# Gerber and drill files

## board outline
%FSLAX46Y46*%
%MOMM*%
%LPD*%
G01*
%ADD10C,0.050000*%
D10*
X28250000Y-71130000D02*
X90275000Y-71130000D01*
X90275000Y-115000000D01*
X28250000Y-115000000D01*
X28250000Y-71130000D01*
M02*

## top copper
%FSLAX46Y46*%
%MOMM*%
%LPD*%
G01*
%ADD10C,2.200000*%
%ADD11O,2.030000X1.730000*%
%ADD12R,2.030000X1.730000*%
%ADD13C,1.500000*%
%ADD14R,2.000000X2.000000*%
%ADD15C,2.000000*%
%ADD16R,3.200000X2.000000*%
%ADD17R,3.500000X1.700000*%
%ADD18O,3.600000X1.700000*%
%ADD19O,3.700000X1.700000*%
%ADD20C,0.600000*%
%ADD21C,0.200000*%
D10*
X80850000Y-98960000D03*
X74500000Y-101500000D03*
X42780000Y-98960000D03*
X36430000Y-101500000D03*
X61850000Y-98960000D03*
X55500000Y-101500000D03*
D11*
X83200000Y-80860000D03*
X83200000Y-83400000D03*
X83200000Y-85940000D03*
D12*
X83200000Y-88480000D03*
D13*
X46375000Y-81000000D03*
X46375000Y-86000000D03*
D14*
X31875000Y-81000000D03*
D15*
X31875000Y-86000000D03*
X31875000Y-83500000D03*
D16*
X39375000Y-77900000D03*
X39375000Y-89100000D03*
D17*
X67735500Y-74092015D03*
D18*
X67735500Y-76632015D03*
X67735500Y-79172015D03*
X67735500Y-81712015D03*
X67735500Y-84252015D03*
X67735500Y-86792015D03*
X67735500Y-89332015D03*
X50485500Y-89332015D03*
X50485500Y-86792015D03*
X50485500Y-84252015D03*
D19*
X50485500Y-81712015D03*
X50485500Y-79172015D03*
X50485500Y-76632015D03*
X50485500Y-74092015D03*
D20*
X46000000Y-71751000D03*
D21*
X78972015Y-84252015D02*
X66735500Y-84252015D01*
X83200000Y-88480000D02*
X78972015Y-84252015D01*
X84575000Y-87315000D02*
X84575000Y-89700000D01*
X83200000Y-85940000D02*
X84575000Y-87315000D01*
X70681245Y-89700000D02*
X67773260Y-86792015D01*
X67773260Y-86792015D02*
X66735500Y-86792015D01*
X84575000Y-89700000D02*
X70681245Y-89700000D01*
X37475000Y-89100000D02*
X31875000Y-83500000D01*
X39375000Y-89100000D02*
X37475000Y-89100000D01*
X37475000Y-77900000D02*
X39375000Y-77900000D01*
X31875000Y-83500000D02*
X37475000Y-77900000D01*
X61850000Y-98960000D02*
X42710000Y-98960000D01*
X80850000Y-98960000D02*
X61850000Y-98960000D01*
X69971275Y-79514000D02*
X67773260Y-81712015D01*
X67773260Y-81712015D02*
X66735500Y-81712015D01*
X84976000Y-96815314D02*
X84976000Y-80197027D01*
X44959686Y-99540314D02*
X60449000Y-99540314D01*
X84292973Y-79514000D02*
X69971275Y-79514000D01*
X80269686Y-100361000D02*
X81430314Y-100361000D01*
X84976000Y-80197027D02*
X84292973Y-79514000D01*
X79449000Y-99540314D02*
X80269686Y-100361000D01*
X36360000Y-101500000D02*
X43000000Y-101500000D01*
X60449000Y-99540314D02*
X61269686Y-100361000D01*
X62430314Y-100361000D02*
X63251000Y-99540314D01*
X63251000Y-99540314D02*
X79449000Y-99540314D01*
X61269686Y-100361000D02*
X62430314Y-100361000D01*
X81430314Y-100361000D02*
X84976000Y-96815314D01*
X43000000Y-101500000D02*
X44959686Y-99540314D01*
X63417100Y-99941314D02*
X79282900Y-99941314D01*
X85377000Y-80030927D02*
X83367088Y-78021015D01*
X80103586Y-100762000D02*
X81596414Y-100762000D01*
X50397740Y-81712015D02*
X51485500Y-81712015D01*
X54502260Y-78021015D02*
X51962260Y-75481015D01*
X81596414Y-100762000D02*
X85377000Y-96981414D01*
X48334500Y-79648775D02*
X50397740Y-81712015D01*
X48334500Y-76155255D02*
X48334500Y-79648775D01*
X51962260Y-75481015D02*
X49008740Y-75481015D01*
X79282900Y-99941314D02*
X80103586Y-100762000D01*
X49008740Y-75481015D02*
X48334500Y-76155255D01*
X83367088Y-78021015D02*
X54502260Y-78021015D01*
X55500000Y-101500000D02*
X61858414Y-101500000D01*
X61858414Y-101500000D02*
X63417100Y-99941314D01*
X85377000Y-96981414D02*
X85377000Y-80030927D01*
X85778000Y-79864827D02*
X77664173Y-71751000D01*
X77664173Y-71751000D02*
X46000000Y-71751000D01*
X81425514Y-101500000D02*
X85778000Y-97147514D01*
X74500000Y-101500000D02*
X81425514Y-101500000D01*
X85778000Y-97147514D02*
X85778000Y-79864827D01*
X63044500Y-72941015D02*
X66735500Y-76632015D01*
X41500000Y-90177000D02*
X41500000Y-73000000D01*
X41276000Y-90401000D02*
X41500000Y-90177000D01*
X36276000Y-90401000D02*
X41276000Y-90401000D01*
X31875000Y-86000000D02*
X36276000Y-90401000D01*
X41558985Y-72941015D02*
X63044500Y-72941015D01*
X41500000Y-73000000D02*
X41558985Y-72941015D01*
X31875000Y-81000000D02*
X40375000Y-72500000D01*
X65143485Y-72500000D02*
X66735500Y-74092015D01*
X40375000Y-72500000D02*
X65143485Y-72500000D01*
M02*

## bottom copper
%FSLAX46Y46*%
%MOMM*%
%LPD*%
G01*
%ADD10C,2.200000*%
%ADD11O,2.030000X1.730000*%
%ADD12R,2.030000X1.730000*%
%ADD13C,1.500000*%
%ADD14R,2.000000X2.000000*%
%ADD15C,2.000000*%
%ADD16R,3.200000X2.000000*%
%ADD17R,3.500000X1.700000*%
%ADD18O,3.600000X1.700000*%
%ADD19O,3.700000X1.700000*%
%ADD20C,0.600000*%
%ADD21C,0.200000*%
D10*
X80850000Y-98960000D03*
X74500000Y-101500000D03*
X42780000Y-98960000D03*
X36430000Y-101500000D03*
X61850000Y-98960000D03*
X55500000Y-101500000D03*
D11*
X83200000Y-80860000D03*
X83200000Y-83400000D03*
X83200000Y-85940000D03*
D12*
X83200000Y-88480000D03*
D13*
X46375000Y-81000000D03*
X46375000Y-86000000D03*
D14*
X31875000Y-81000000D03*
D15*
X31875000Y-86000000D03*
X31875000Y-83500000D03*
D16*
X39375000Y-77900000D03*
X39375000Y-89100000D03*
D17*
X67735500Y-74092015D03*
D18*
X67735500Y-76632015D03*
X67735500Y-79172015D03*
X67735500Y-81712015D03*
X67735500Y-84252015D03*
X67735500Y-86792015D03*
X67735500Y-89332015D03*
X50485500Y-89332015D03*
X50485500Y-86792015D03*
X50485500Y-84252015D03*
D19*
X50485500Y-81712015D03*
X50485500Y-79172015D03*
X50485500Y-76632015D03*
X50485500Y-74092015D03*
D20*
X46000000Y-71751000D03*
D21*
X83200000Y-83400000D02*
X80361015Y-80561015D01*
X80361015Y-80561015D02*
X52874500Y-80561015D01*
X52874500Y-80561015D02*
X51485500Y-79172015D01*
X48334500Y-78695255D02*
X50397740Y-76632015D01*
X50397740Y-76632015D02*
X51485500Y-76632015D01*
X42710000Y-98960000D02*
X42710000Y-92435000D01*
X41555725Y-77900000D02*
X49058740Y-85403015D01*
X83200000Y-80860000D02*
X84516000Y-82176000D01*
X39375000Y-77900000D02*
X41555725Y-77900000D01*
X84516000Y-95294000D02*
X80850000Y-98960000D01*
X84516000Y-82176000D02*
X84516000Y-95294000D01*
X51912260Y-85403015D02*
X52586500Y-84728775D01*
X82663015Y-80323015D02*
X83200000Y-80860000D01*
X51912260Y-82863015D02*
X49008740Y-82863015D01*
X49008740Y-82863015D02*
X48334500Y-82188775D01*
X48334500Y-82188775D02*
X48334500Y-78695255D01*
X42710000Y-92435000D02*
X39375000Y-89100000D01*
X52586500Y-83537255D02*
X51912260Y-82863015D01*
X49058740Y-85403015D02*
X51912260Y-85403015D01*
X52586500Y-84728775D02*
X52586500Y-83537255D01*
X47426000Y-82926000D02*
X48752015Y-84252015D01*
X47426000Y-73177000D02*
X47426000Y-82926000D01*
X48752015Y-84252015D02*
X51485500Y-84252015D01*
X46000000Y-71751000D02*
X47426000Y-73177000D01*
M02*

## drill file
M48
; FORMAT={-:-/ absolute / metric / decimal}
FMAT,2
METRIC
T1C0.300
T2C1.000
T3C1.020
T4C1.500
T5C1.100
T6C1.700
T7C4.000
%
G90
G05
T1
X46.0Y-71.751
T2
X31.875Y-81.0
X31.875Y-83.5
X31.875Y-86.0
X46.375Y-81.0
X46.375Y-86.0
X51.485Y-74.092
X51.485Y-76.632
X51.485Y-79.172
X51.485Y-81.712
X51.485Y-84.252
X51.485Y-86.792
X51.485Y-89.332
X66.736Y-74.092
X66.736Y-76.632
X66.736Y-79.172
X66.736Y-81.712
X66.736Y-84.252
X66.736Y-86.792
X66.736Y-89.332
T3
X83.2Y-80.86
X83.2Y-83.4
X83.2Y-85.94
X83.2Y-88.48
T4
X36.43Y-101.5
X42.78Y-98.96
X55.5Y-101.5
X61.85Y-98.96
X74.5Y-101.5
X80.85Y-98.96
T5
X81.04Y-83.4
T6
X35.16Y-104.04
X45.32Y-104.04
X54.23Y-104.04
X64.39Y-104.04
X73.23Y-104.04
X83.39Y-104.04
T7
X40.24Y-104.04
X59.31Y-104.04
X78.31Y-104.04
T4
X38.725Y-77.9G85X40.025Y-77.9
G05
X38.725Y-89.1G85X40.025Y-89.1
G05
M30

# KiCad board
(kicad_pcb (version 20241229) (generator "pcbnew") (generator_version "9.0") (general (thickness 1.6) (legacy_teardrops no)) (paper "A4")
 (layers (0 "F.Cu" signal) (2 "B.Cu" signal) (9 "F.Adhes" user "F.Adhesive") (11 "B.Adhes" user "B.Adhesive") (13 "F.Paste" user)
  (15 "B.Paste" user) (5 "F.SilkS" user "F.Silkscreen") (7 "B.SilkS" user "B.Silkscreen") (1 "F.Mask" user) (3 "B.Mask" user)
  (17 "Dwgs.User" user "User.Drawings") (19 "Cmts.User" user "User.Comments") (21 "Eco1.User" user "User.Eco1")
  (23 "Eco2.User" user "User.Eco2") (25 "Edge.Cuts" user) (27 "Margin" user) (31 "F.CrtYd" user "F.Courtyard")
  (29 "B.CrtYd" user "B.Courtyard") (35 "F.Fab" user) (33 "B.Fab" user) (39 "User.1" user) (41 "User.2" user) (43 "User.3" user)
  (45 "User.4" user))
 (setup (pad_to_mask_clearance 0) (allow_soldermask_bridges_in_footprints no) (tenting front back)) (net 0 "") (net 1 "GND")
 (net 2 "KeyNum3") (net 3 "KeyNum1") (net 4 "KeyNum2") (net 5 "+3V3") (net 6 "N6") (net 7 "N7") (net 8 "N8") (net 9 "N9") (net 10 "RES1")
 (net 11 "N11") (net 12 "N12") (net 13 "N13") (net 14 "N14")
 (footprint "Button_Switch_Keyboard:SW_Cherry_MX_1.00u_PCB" (layer "F.Cu") (at 80.85 98.96)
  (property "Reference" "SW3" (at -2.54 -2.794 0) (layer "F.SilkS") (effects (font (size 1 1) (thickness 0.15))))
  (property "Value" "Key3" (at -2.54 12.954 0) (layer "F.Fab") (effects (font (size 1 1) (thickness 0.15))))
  (pad "" np_thru_hole circle (at -7.62 5.08) (size 1.7 1.7) (drill 1.7) (layers "*.Cu" "*.Mask"))
  (pad "" np_thru_hole circle (at -2.54 5.08) (size 4 4) (drill 4) (layers "*.Cu" "*.Mask"))
  (pad "" np_thru_hole circle (at 2.54 5.08) (size 1.7 1.7) (drill 1.7) (layers "*.Cu" "*.Mask"))
  (pad "1" thru_hole circle (at 0 0) (size 2.2 2.2) (drill 1.5) (layers "*.Cu" "*.Mask") (remove_unused_layers no) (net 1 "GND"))
  (pad "2" thru_hole circle (at -6.35 2.54) (size 2.2 2.2) (drill 1.5) (layers "*.Cu" "*.Mask") (remove_unused_layers no) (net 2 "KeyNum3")))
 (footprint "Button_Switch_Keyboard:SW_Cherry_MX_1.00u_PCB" (layer "F.Cu") (at 42.78 98.96)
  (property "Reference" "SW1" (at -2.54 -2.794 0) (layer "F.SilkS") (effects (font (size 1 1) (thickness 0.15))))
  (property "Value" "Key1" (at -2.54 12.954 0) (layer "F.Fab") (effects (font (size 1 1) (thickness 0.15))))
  (pad "" np_thru_hole circle (at -7.62 5.08) (size 1.7 1.7) (drill 1.7) (layers "*.Cu" "*.Mask"))
  (pad "" np_thru_hole circle (at -2.54 5.08) (size 4 4) (drill 4) (layers "*.Cu" "*.Mask"))
  (pad "" np_thru_hole circle (at 2.54 5.08) (size 1.7 1.7) (drill 1.7) (layers "*.Cu" "*.Mask"))
  (pad "1" thru_hole circle (at 0 0) (size 2.2 2.2) (drill 1.5) (layers "*.Cu" "*.Mask") (remove_unused_layers no) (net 1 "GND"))
  (pad "2" thru_hole circle (at -6.35 2.54) (size 2.2 2.2) (drill 1.5) (layers "*.Cu" "*.Mask") (remove_unused_layers no) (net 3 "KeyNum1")))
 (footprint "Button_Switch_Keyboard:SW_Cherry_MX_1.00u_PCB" (layer "F.Cu") (at 61.85 98.96)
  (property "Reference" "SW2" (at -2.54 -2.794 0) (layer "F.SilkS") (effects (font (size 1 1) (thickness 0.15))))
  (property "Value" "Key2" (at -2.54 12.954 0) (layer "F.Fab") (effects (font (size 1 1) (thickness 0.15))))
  (pad "" np_thru_hole circle (at -7.62 5.08) (size 1.7 1.7) (drill 1.7) (layers "*.Cu" "*.Mask"))
  (pad "" np_thru_hole circle (at -2.54 5.08) (size 4 4) (drill 4) (layers "*.Cu" "*.Mask"))
  (pad "" np_thru_hole circle (at 2.54 5.08) (size 1.7 1.7) (drill 1.7) (layers "*.Cu" "*.Mask"))
  (pad "1" thru_hole circle (at 0 0) (size 2.2 2.2) (drill 1.5) (layers "*.Cu" "*.Mask") (remove_unused_layers no) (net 1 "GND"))
  (pad "2" thru_hole circle (at -6.35 2.54) (size 2.2 2.2) (drill 1.5) (layers "*.Cu" "*.Mask") (remove_unused_layers no) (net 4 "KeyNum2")))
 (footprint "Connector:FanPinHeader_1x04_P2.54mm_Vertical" (layer "F.Cu") (at 83.2 88.48 90)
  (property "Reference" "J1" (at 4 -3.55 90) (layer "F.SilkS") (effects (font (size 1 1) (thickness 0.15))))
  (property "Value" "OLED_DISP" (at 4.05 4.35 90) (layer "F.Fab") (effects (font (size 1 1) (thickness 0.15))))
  (pad "" np_thru_hole circle (at 5.08 -2.16 180) (size 1.1 1.1) (drill 1.1) (layers "*.Cu" "*.Mask"))
  (pad "1" thru_hole oval (at 7.62 0 180) (size 2.03 1.73) (drill 1.02) (layers "*.Cu" "*.Mask") (remove_unused_layers no) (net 1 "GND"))
  (pad "2" thru_hole oval (at 5.08 0 180) (size 2.03 1.73) (drill 1.02) (layers "*.Cu" "*.Mask") (remove_unused_layers no) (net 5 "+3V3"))
  (pad "3" thru_hole oval (at 2.54 0 180) (size 2.03 1.73) (drill 1.02) (layers "*.Cu" "*.Mask") (remove_unused_layers no) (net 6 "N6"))
  (pad "4" thru_hole rect (at 0 0 180) (size 2.03 1.73) (drill 1.02) (layers "*.Cu" "*.Mask") (remove_unused_layers no) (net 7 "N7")))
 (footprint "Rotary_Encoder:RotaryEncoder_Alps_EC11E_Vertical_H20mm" (layer "F.Cu") (at 31.875 81)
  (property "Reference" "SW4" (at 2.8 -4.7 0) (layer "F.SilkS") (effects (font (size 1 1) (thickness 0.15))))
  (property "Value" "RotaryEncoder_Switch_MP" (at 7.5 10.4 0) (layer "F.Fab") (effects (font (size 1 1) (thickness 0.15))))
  (pad "" thru_hole circle (at 14.5 0) (size 1.5 1.5) (drill 1) (layers "*.Cu" "*.Mask") (remove_unused_layers no))
  (pad "" thru_hole circle (at 14.5 5) (size 1.5 1.5) (drill 1) (layers "*.Cu" "*.Mask") (remove_unused_layers no))
  (pad "A" thru_hole rect (at 0 0) (size 2 2) (drill 1) (layers "*.Cu" "*.Mask") (remove_unused_layers no) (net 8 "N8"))
  (pad "B" thru_hole circle (at 0 5) (size 2 2) (drill 1) (layers "*.Cu" "*.Mask") (remove_unused_layers no) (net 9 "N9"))
  (pad "C" thru_hole circle (at 0 2.5) (size 2 2) (drill 1) (layers "*.Cu" "*.Mask") (remove_unused_layers no) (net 1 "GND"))
  (pad "MP" thru_hole rect (at 7.5 -3.1) (size 3.2 2) (drill oval 2.8 1.5) (layers "*.Cu" "*.Mask") (remove_unused_layers no) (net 1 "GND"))
  (pad "MP" thru_hole rect (at 7.5 8.1) (size 3.2 2) (drill oval 2.8 1.5) (layers "*.Cu" "*.Mask") (remove_unused_layers no) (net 1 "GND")))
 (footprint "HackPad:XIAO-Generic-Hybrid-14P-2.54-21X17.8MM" (layer "B.Cu") (at 59.1105 81.712015 180)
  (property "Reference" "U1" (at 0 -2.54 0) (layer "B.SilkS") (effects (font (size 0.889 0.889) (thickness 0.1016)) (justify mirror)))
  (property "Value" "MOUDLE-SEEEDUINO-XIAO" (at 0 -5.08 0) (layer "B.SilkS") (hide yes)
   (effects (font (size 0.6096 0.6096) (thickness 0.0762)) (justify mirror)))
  (pad "1" thru_hole rect (at -7.625 7.62 180) (size 3.5 1.7) (drill 1 (offset -1 0)) (layers "*.Cu" "*.Mask") (remove_unused_layers no)
   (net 8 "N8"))
  (pad "2" thru_hole oval (at -7.625 5.08 180) (size 3.6 1.7) (drill 1 (offset -1 0)) (layers "*.Cu" "*.Mask") (remove_unused_layers no)
   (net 9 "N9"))
  (pad "3" thru_hole oval (at -7.625 2.54 180) (size 3.6 1.7) (drill 1 (offset -1 0)) (layers "*.Cu" "*.Mask") (remove_unused_layers no)
   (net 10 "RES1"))
  (pad "4" thru_hole oval (at -7.625 0 180) (size 3.6 1.7) (drill 1 (offset -1 0)) (layers "*.Cu" "*.Mask") (remove_unused_layers no)
   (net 3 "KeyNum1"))
  (pad "5" thru_hole oval (at -7.625 -2.54 180) (size 3.6 1.7) (drill 1 (offset -1 0)) (layers "*.Cu" "*.Mask") (remove_unused_layers no)
   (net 7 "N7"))
  (pad "6" thru_hole oval (at -7.625 -5.08) (size 3.6 1.7) (drill 1 (offset 1 0)) (layers "*.Cu" "*.Mask") (remove_unused_layers no)
   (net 6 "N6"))
  (pad "7" thru_hole oval (at -7.625 -7.62 180) (size 3.6 1.7) (drill 1 (offset -1 0)) (layers "*.Cu" "*.Mask") (remove_unused_layers no)
   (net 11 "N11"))
  (pad "8" thru_hole oval (at 7.625 -7.62 180) (size 3.6 1.7) (drill 1 (offset 1 0)) (layers "*.Cu" "*.Mask") (remove_unused_layers no)
   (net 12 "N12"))
  (pad "9" thru_hole oval (at 7.625 -5.08 180) (size 3.6 1.7) (drill 1 (offset 1 0)) (layers "*.Cu" "*.Mask") (remove_unused_layers no)
   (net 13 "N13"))
  (pad "10" thru_hole oval (at 7.625 -2.54 180) (size 3.6 1.7) (drill 1 (offset 1 0)) (layers "*.Cu" "*.Mask") (remove_unused_layers no)
   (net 2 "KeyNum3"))
  (pad "11" thru_hole oval (at 7.625 0 180) (size 3.7 1.7) (drill 1 (offset 1 0)) (layers "*.Cu" "*.Mask") (remove_unused_layers no)
   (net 4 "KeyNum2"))
  (pad "12" thru_hole oval (at 7.625 2.54 180) (size 3.7 1.7) (drill 1 (offset 1 0)) (layers "*.Cu" "*.Mask") (remove_unused_layers no)
   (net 5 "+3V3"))
  (pad "13" thru_hole oval (at 7.625 5.08 180) (size 3.7 1.7) (drill 1 (offset 1 0)) (layers "*.Cu" "*.Mask") (remove_unused_layers no)
   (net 1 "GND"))
  (pad "14" thru_hole oval (at 7.625 7.62 180) (size 3.7 1.7) (drill 1 (offset 1 0)) (layers "*.Cu" "*.Mask") (remove_unused_layers no)
   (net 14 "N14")))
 (gr_rect (start 28.25 71.13) (end 90.275 115) (stroke (width 0.05) (type default)) (fill no) (layer "Edge.Cuts"))
 (segment (start 78.972015 84.252015) (end 66.7355 84.252015) (width 0.2) (layer "F.Cu") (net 7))
 (segment (start 83.2 88.48) (end 78.972015 84.252015) (width 0.2) (layer "F.Cu") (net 7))
 (segment (start 83.2 83.4) (end 80.361015 80.561015) (width 0.2) (layer "B.Cu") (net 5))
 (segment (start 80.361015 80.561015) (end 52.8745 80.561015) (width 0.2) (layer "B.Cu") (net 5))
 (segment (start 52.8745 80.561015) (end 51.4855 79.172015) (width 0.2) (layer "B.Cu") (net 5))
 (segment (start 84.575 87.315) (end 84.575 89.7) (width 0.2) (layer "F.Cu") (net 6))
 (segment (start 83.2 85.94) (end 84.575 87.315) (width 0.2) (layer "F.Cu") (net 6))
 (segment (start 70.681245 89.7) (end 67.77326 86.792015) (width 0.2) (layer "F.Cu") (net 6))
 (segment (start 67.77326 86.792015) (end 66.7355 86.792015) (width 0.2) (layer "F.Cu") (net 6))
 (segment (start 84.575 89.7) (end 70.681245 89.7) (width 0.2) (layer "F.Cu") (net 6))
 (segment (start 37.475 89.1) (end 31.875 83.5) (width 0.2) (layer "F.Cu") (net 1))
 (segment (start 39.375 89.1) (end 37.475 89.1) (width 0.2) (layer "F.Cu") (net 1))
 (segment (start 37.475 77.9) (end 39.375 77.9) (width 0.2) (layer "F.Cu") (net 1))
 (segment (start 31.875 83.5) (end 37.475 77.9) (width 0.2) (layer "F.Cu") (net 1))
 (segment (start 61.85 98.96) (end 42.71 98.96) (width 0.2) (layer "F.Cu") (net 1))
 (segment (start 80.85 98.96) (end 61.85 98.96) (width 0.2) (layer "F.Cu") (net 1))
 (segment (start 48.3345 78.695255) (end 50.39774 76.632015) (width 0.2) (layer "B.Cu") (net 1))
 (segment (start 50.39774 76.632015) (end 51.4855 76.632015) (width 0.2) (layer "B.Cu") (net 1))
 (segment (start 42.71 98.96) (end 42.71 92.435) (width 0.2) (layer "B.Cu") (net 1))
 (segment (start 41.555725 77.9) (end 49.05874 85.403015) (width 0.2) (layer "B.Cu") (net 1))
 (segment (start 83.2 80.86) (end 84.516 82.176) (width 0.2) (layer "B.Cu") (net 1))
 (segment (start 39.375 77.9) (end 41.555725 77.9) (width 0.2) (layer "B.Cu") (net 1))
 (segment (start 84.516 95.294) (end 80.85 98.96) (width 0.2) (layer "B.Cu") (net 1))
 (segment (start 84.516 82.176) (end 84.516 95.294) (width 0.2) (layer "B.Cu") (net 1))
 (segment (start 51.91226 85.403015) (end 52.5865 84.728775) (width 0.2) (layer "B.Cu") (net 1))
 (segment (start 82.663015 80.323015) (end 83.2 80.86) (width 0.2) (layer "B.Cu") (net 1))
 (segment (start 51.91226 82.863015) (end 49.00874 82.863015) (width 0.2) (layer "B.Cu") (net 1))
 (segment (start 49.00874 82.863015) (end 48.3345 82.188775) (width 0.2) (layer "B.Cu") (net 1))
 (segment (start 48.3345 82.188775) (end 48.3345 78.695255) (width 0.2) (layer "B.Cu") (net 1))
 (segment (start 42.71 92.435) (end 39.375 89.1) (width 0.2) (layer "B.Cu") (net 1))
 (segment (start 52.5865 83.537255) (end 51.91226 82.863015) (width 0.2) (layer "B.Cu") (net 1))
 (segment (start 49.05874 85.403015) (end 51.91226 85.403015) (width 0.2) (layer "B.Cu") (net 1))
 (segment (start 52.5865 84.728775) (end 52.5865 83.537255) (width 0.2) (layer "B.Cu") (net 1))
 (segment (start 69.971275 79.514) (end 67.77326 81.712015) (width 0.2) (layer "F.Cu") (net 3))
 (segment (start 67.77326 81.712015) (end 66.7355 81.712015) (width 0.2) (layer "F.Cu") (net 3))
 (segment (start 84.976 96.815314) (end 84.976 80.197027) (width 0.2) (layer "F.Cu") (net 3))
 (segment (start 44.959686 99.540314) (end 60.449 99.540314) (width 0.2) (layer "F.Cu") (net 3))
 (segment (start 84.292973 79.514) (end 69.971275 79.514) (width 0.2) (layer "F.Cu") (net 3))
 (segment (start 80.269686 100.361) (end 81.430314 100.361) (width 0.2) (layer "F.Cu") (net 3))
 (segment (start 84.976 80.197027) (end 84.292973 79.514) (width 0.2) (layer "F.Cu") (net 3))
 (segment (start 79.449 99.540314) (end 80.269686 100.361) (width 0.2) (layer "F.Cu") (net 3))
 (segment (start 36.36 101.5) (end 43 101.5) (width 0.2) (layer "F.Cu") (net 3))
 (segment (start 60.449 99.540314) (end 61.269686 100.361) (width 0.2) (layer "F.Cu") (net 3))
 (segment (start 62.430314 100.361) (end 63.251 99.540314) (width 0.2) (layer "F.Cu") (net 3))
 (segment (start 63.251 99.540314) (end 79.449 99.540314) (width 0.2) (layer "F.Cu") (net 3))
 (segment (start 61.269686 100.361) (end 62.430314 100.361) (width 0.2) (layer "F.Cu") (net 3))
 (segment (start 81.430314 100.361) (end 84.976 96.815314) (width 0.2) (layer "F.Cu") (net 3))
 (segment (start 43 101.5) (end 44.959686 99.540314) (width 0.2) (layer "F.Cu") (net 3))
 (segment (start 63.4171 99.941314) (end 79.2829 99.941314) (width 0.2) (layer "F.Cu") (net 4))
 (segment (start 85.377 80.030927) (end 83.367088 78.021015) (width 0.2) (layer "F.Cu") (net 4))
 (segment (start 80.103586 100.762) (end 81.596414 100.762) (width 0.2) (layer "F.Cu") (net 4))
 (segment (start 50.39774 81.712015) (end 51.4855 81.712015) (width 0.2) (layer "F.Cu") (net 4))
 (segment (start 54.50226 78.021015) (end 51.96226 75.481015) (width 0.2) (layer "F.Cu") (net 4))
 (segment (start 81.596414 100.762) (end 85.377 96.981414) (width 0.2) (layer "F.Cu") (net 4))
 (segment (start 48.3345 79.648775) (end 50.39774 81.712015) (width 0.2) (layer "F.Cu") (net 4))
 (segment (start 48.3345 76.155255) (end 48.3345 79.648775) (width 0.2) (layer "F.Cu") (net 4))
 (segment (start 51.96226 75.481015) (end 49.00874 75.481015) (width 0.2) (layer "F.Cu") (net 4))
 (segment (start 79.2829 99.941314) (end 80.103586 100.762) (width 0.2) (layer "F.Cu") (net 4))
 (segment (start 49.00874 75.481015) (end 48.3345 76.155255) (width 0.2) (layer "F.Cu") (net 4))
 (segment (start 83.367088 78.021015) (end 54.50226 78.021015) (width 0.2) (layer "F.Cu") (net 4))
 (segment (start 55.5 101.5) (end 61.858414 101.5) (width 0.2) (layer "F.Cu") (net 4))
 (segment (start 61.858414 101.5) (end 63.4171 99.941314) (width 0.2) (layer "F.Cu") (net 4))
 (segment (start 85.377 96.981414) (end 85.377 80.030927) (width 0.2) (layer "F.Cu") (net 4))
 (segment (start 85.778 79.864827) (end 77.664173 71.751) (width 0.2) (layer "F.Cu") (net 2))
 (segment (start 77.664173 71.751) (end 46 71.751) (width 0.2) (layer "F.Cu") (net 2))
 (segment (start 81.425514 101.5) (end 85.778 97.147514) (width 0.2) (layer "F.Cu") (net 2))
 (segment (start 74.5 101.5) (end 81.425514 101.5) (width 0.2) (layer "F.Cu") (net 2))
 (segment (start 85.778 97.147514) (end 85.778 79.864827) (width 0.2) (layer "F.Cu") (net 2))
 (via (at 46 71.751) (size 0.6) (drill 0.3) (layers "F.Cu" "B.Cu") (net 2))
 (segment (start 47.426 82.926) (end 48.752015 84.252015) (width 0.2) (layer "B.Cu") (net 2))
 (segment (start 47.426 73.177) (end 47.426 82.926) (width 0.2) (layer "B.Cu") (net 2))
 (segment (start 48.752015 84.252015) (end 51.4855 84.252015) (width 0.2) (layer "B.Cu") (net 2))
 (segment (start 46 71.751) (end 47.426 73.177) (width 0.2) (layer "B.Cu") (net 2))
 (segment (start 63.0445 72.941015) (end 66.7355 76.632015) (width 0.2) (layer "F.Cu") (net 9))
 (segment (start 41.5 90.177) (end 41.5 73) (width 0.2) (layer "F.Cu") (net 9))
 (segment (start 41.276 90.401) (end 41.5 90.177) (width 0.2) (layer "F.Cu") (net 9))
 (segment (start 36.276 90.401) (end 41.276 90.401) (width 0.2) (layer "F.Cu") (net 9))
 (segment (start 31.875 86) (end 36.276 90.401) (width 0.2) (layer "F.Cu") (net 9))
 (segment (start 41.558985 72.941015) (end 63.0445 72.941015) (width 0.2) (layer "F.Cu") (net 9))
 (segment (start 41.5 73) (end 41.558985 72.941015) (width 0.2) (layer "F.Cu") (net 9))
 (segment (start 31.875 81) (end 40.375 72.5) (width 0.2) (layer "F.Cu") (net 8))
 (segment (start 65.143485 72.5) (end 66.7355 74.092015) (width 0.2) (layer "F.Cu") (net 8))
 (segment (start 40.375 72.5) (end 65.143485 72.5) (width 0.2) (layer "F.Cu") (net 8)))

